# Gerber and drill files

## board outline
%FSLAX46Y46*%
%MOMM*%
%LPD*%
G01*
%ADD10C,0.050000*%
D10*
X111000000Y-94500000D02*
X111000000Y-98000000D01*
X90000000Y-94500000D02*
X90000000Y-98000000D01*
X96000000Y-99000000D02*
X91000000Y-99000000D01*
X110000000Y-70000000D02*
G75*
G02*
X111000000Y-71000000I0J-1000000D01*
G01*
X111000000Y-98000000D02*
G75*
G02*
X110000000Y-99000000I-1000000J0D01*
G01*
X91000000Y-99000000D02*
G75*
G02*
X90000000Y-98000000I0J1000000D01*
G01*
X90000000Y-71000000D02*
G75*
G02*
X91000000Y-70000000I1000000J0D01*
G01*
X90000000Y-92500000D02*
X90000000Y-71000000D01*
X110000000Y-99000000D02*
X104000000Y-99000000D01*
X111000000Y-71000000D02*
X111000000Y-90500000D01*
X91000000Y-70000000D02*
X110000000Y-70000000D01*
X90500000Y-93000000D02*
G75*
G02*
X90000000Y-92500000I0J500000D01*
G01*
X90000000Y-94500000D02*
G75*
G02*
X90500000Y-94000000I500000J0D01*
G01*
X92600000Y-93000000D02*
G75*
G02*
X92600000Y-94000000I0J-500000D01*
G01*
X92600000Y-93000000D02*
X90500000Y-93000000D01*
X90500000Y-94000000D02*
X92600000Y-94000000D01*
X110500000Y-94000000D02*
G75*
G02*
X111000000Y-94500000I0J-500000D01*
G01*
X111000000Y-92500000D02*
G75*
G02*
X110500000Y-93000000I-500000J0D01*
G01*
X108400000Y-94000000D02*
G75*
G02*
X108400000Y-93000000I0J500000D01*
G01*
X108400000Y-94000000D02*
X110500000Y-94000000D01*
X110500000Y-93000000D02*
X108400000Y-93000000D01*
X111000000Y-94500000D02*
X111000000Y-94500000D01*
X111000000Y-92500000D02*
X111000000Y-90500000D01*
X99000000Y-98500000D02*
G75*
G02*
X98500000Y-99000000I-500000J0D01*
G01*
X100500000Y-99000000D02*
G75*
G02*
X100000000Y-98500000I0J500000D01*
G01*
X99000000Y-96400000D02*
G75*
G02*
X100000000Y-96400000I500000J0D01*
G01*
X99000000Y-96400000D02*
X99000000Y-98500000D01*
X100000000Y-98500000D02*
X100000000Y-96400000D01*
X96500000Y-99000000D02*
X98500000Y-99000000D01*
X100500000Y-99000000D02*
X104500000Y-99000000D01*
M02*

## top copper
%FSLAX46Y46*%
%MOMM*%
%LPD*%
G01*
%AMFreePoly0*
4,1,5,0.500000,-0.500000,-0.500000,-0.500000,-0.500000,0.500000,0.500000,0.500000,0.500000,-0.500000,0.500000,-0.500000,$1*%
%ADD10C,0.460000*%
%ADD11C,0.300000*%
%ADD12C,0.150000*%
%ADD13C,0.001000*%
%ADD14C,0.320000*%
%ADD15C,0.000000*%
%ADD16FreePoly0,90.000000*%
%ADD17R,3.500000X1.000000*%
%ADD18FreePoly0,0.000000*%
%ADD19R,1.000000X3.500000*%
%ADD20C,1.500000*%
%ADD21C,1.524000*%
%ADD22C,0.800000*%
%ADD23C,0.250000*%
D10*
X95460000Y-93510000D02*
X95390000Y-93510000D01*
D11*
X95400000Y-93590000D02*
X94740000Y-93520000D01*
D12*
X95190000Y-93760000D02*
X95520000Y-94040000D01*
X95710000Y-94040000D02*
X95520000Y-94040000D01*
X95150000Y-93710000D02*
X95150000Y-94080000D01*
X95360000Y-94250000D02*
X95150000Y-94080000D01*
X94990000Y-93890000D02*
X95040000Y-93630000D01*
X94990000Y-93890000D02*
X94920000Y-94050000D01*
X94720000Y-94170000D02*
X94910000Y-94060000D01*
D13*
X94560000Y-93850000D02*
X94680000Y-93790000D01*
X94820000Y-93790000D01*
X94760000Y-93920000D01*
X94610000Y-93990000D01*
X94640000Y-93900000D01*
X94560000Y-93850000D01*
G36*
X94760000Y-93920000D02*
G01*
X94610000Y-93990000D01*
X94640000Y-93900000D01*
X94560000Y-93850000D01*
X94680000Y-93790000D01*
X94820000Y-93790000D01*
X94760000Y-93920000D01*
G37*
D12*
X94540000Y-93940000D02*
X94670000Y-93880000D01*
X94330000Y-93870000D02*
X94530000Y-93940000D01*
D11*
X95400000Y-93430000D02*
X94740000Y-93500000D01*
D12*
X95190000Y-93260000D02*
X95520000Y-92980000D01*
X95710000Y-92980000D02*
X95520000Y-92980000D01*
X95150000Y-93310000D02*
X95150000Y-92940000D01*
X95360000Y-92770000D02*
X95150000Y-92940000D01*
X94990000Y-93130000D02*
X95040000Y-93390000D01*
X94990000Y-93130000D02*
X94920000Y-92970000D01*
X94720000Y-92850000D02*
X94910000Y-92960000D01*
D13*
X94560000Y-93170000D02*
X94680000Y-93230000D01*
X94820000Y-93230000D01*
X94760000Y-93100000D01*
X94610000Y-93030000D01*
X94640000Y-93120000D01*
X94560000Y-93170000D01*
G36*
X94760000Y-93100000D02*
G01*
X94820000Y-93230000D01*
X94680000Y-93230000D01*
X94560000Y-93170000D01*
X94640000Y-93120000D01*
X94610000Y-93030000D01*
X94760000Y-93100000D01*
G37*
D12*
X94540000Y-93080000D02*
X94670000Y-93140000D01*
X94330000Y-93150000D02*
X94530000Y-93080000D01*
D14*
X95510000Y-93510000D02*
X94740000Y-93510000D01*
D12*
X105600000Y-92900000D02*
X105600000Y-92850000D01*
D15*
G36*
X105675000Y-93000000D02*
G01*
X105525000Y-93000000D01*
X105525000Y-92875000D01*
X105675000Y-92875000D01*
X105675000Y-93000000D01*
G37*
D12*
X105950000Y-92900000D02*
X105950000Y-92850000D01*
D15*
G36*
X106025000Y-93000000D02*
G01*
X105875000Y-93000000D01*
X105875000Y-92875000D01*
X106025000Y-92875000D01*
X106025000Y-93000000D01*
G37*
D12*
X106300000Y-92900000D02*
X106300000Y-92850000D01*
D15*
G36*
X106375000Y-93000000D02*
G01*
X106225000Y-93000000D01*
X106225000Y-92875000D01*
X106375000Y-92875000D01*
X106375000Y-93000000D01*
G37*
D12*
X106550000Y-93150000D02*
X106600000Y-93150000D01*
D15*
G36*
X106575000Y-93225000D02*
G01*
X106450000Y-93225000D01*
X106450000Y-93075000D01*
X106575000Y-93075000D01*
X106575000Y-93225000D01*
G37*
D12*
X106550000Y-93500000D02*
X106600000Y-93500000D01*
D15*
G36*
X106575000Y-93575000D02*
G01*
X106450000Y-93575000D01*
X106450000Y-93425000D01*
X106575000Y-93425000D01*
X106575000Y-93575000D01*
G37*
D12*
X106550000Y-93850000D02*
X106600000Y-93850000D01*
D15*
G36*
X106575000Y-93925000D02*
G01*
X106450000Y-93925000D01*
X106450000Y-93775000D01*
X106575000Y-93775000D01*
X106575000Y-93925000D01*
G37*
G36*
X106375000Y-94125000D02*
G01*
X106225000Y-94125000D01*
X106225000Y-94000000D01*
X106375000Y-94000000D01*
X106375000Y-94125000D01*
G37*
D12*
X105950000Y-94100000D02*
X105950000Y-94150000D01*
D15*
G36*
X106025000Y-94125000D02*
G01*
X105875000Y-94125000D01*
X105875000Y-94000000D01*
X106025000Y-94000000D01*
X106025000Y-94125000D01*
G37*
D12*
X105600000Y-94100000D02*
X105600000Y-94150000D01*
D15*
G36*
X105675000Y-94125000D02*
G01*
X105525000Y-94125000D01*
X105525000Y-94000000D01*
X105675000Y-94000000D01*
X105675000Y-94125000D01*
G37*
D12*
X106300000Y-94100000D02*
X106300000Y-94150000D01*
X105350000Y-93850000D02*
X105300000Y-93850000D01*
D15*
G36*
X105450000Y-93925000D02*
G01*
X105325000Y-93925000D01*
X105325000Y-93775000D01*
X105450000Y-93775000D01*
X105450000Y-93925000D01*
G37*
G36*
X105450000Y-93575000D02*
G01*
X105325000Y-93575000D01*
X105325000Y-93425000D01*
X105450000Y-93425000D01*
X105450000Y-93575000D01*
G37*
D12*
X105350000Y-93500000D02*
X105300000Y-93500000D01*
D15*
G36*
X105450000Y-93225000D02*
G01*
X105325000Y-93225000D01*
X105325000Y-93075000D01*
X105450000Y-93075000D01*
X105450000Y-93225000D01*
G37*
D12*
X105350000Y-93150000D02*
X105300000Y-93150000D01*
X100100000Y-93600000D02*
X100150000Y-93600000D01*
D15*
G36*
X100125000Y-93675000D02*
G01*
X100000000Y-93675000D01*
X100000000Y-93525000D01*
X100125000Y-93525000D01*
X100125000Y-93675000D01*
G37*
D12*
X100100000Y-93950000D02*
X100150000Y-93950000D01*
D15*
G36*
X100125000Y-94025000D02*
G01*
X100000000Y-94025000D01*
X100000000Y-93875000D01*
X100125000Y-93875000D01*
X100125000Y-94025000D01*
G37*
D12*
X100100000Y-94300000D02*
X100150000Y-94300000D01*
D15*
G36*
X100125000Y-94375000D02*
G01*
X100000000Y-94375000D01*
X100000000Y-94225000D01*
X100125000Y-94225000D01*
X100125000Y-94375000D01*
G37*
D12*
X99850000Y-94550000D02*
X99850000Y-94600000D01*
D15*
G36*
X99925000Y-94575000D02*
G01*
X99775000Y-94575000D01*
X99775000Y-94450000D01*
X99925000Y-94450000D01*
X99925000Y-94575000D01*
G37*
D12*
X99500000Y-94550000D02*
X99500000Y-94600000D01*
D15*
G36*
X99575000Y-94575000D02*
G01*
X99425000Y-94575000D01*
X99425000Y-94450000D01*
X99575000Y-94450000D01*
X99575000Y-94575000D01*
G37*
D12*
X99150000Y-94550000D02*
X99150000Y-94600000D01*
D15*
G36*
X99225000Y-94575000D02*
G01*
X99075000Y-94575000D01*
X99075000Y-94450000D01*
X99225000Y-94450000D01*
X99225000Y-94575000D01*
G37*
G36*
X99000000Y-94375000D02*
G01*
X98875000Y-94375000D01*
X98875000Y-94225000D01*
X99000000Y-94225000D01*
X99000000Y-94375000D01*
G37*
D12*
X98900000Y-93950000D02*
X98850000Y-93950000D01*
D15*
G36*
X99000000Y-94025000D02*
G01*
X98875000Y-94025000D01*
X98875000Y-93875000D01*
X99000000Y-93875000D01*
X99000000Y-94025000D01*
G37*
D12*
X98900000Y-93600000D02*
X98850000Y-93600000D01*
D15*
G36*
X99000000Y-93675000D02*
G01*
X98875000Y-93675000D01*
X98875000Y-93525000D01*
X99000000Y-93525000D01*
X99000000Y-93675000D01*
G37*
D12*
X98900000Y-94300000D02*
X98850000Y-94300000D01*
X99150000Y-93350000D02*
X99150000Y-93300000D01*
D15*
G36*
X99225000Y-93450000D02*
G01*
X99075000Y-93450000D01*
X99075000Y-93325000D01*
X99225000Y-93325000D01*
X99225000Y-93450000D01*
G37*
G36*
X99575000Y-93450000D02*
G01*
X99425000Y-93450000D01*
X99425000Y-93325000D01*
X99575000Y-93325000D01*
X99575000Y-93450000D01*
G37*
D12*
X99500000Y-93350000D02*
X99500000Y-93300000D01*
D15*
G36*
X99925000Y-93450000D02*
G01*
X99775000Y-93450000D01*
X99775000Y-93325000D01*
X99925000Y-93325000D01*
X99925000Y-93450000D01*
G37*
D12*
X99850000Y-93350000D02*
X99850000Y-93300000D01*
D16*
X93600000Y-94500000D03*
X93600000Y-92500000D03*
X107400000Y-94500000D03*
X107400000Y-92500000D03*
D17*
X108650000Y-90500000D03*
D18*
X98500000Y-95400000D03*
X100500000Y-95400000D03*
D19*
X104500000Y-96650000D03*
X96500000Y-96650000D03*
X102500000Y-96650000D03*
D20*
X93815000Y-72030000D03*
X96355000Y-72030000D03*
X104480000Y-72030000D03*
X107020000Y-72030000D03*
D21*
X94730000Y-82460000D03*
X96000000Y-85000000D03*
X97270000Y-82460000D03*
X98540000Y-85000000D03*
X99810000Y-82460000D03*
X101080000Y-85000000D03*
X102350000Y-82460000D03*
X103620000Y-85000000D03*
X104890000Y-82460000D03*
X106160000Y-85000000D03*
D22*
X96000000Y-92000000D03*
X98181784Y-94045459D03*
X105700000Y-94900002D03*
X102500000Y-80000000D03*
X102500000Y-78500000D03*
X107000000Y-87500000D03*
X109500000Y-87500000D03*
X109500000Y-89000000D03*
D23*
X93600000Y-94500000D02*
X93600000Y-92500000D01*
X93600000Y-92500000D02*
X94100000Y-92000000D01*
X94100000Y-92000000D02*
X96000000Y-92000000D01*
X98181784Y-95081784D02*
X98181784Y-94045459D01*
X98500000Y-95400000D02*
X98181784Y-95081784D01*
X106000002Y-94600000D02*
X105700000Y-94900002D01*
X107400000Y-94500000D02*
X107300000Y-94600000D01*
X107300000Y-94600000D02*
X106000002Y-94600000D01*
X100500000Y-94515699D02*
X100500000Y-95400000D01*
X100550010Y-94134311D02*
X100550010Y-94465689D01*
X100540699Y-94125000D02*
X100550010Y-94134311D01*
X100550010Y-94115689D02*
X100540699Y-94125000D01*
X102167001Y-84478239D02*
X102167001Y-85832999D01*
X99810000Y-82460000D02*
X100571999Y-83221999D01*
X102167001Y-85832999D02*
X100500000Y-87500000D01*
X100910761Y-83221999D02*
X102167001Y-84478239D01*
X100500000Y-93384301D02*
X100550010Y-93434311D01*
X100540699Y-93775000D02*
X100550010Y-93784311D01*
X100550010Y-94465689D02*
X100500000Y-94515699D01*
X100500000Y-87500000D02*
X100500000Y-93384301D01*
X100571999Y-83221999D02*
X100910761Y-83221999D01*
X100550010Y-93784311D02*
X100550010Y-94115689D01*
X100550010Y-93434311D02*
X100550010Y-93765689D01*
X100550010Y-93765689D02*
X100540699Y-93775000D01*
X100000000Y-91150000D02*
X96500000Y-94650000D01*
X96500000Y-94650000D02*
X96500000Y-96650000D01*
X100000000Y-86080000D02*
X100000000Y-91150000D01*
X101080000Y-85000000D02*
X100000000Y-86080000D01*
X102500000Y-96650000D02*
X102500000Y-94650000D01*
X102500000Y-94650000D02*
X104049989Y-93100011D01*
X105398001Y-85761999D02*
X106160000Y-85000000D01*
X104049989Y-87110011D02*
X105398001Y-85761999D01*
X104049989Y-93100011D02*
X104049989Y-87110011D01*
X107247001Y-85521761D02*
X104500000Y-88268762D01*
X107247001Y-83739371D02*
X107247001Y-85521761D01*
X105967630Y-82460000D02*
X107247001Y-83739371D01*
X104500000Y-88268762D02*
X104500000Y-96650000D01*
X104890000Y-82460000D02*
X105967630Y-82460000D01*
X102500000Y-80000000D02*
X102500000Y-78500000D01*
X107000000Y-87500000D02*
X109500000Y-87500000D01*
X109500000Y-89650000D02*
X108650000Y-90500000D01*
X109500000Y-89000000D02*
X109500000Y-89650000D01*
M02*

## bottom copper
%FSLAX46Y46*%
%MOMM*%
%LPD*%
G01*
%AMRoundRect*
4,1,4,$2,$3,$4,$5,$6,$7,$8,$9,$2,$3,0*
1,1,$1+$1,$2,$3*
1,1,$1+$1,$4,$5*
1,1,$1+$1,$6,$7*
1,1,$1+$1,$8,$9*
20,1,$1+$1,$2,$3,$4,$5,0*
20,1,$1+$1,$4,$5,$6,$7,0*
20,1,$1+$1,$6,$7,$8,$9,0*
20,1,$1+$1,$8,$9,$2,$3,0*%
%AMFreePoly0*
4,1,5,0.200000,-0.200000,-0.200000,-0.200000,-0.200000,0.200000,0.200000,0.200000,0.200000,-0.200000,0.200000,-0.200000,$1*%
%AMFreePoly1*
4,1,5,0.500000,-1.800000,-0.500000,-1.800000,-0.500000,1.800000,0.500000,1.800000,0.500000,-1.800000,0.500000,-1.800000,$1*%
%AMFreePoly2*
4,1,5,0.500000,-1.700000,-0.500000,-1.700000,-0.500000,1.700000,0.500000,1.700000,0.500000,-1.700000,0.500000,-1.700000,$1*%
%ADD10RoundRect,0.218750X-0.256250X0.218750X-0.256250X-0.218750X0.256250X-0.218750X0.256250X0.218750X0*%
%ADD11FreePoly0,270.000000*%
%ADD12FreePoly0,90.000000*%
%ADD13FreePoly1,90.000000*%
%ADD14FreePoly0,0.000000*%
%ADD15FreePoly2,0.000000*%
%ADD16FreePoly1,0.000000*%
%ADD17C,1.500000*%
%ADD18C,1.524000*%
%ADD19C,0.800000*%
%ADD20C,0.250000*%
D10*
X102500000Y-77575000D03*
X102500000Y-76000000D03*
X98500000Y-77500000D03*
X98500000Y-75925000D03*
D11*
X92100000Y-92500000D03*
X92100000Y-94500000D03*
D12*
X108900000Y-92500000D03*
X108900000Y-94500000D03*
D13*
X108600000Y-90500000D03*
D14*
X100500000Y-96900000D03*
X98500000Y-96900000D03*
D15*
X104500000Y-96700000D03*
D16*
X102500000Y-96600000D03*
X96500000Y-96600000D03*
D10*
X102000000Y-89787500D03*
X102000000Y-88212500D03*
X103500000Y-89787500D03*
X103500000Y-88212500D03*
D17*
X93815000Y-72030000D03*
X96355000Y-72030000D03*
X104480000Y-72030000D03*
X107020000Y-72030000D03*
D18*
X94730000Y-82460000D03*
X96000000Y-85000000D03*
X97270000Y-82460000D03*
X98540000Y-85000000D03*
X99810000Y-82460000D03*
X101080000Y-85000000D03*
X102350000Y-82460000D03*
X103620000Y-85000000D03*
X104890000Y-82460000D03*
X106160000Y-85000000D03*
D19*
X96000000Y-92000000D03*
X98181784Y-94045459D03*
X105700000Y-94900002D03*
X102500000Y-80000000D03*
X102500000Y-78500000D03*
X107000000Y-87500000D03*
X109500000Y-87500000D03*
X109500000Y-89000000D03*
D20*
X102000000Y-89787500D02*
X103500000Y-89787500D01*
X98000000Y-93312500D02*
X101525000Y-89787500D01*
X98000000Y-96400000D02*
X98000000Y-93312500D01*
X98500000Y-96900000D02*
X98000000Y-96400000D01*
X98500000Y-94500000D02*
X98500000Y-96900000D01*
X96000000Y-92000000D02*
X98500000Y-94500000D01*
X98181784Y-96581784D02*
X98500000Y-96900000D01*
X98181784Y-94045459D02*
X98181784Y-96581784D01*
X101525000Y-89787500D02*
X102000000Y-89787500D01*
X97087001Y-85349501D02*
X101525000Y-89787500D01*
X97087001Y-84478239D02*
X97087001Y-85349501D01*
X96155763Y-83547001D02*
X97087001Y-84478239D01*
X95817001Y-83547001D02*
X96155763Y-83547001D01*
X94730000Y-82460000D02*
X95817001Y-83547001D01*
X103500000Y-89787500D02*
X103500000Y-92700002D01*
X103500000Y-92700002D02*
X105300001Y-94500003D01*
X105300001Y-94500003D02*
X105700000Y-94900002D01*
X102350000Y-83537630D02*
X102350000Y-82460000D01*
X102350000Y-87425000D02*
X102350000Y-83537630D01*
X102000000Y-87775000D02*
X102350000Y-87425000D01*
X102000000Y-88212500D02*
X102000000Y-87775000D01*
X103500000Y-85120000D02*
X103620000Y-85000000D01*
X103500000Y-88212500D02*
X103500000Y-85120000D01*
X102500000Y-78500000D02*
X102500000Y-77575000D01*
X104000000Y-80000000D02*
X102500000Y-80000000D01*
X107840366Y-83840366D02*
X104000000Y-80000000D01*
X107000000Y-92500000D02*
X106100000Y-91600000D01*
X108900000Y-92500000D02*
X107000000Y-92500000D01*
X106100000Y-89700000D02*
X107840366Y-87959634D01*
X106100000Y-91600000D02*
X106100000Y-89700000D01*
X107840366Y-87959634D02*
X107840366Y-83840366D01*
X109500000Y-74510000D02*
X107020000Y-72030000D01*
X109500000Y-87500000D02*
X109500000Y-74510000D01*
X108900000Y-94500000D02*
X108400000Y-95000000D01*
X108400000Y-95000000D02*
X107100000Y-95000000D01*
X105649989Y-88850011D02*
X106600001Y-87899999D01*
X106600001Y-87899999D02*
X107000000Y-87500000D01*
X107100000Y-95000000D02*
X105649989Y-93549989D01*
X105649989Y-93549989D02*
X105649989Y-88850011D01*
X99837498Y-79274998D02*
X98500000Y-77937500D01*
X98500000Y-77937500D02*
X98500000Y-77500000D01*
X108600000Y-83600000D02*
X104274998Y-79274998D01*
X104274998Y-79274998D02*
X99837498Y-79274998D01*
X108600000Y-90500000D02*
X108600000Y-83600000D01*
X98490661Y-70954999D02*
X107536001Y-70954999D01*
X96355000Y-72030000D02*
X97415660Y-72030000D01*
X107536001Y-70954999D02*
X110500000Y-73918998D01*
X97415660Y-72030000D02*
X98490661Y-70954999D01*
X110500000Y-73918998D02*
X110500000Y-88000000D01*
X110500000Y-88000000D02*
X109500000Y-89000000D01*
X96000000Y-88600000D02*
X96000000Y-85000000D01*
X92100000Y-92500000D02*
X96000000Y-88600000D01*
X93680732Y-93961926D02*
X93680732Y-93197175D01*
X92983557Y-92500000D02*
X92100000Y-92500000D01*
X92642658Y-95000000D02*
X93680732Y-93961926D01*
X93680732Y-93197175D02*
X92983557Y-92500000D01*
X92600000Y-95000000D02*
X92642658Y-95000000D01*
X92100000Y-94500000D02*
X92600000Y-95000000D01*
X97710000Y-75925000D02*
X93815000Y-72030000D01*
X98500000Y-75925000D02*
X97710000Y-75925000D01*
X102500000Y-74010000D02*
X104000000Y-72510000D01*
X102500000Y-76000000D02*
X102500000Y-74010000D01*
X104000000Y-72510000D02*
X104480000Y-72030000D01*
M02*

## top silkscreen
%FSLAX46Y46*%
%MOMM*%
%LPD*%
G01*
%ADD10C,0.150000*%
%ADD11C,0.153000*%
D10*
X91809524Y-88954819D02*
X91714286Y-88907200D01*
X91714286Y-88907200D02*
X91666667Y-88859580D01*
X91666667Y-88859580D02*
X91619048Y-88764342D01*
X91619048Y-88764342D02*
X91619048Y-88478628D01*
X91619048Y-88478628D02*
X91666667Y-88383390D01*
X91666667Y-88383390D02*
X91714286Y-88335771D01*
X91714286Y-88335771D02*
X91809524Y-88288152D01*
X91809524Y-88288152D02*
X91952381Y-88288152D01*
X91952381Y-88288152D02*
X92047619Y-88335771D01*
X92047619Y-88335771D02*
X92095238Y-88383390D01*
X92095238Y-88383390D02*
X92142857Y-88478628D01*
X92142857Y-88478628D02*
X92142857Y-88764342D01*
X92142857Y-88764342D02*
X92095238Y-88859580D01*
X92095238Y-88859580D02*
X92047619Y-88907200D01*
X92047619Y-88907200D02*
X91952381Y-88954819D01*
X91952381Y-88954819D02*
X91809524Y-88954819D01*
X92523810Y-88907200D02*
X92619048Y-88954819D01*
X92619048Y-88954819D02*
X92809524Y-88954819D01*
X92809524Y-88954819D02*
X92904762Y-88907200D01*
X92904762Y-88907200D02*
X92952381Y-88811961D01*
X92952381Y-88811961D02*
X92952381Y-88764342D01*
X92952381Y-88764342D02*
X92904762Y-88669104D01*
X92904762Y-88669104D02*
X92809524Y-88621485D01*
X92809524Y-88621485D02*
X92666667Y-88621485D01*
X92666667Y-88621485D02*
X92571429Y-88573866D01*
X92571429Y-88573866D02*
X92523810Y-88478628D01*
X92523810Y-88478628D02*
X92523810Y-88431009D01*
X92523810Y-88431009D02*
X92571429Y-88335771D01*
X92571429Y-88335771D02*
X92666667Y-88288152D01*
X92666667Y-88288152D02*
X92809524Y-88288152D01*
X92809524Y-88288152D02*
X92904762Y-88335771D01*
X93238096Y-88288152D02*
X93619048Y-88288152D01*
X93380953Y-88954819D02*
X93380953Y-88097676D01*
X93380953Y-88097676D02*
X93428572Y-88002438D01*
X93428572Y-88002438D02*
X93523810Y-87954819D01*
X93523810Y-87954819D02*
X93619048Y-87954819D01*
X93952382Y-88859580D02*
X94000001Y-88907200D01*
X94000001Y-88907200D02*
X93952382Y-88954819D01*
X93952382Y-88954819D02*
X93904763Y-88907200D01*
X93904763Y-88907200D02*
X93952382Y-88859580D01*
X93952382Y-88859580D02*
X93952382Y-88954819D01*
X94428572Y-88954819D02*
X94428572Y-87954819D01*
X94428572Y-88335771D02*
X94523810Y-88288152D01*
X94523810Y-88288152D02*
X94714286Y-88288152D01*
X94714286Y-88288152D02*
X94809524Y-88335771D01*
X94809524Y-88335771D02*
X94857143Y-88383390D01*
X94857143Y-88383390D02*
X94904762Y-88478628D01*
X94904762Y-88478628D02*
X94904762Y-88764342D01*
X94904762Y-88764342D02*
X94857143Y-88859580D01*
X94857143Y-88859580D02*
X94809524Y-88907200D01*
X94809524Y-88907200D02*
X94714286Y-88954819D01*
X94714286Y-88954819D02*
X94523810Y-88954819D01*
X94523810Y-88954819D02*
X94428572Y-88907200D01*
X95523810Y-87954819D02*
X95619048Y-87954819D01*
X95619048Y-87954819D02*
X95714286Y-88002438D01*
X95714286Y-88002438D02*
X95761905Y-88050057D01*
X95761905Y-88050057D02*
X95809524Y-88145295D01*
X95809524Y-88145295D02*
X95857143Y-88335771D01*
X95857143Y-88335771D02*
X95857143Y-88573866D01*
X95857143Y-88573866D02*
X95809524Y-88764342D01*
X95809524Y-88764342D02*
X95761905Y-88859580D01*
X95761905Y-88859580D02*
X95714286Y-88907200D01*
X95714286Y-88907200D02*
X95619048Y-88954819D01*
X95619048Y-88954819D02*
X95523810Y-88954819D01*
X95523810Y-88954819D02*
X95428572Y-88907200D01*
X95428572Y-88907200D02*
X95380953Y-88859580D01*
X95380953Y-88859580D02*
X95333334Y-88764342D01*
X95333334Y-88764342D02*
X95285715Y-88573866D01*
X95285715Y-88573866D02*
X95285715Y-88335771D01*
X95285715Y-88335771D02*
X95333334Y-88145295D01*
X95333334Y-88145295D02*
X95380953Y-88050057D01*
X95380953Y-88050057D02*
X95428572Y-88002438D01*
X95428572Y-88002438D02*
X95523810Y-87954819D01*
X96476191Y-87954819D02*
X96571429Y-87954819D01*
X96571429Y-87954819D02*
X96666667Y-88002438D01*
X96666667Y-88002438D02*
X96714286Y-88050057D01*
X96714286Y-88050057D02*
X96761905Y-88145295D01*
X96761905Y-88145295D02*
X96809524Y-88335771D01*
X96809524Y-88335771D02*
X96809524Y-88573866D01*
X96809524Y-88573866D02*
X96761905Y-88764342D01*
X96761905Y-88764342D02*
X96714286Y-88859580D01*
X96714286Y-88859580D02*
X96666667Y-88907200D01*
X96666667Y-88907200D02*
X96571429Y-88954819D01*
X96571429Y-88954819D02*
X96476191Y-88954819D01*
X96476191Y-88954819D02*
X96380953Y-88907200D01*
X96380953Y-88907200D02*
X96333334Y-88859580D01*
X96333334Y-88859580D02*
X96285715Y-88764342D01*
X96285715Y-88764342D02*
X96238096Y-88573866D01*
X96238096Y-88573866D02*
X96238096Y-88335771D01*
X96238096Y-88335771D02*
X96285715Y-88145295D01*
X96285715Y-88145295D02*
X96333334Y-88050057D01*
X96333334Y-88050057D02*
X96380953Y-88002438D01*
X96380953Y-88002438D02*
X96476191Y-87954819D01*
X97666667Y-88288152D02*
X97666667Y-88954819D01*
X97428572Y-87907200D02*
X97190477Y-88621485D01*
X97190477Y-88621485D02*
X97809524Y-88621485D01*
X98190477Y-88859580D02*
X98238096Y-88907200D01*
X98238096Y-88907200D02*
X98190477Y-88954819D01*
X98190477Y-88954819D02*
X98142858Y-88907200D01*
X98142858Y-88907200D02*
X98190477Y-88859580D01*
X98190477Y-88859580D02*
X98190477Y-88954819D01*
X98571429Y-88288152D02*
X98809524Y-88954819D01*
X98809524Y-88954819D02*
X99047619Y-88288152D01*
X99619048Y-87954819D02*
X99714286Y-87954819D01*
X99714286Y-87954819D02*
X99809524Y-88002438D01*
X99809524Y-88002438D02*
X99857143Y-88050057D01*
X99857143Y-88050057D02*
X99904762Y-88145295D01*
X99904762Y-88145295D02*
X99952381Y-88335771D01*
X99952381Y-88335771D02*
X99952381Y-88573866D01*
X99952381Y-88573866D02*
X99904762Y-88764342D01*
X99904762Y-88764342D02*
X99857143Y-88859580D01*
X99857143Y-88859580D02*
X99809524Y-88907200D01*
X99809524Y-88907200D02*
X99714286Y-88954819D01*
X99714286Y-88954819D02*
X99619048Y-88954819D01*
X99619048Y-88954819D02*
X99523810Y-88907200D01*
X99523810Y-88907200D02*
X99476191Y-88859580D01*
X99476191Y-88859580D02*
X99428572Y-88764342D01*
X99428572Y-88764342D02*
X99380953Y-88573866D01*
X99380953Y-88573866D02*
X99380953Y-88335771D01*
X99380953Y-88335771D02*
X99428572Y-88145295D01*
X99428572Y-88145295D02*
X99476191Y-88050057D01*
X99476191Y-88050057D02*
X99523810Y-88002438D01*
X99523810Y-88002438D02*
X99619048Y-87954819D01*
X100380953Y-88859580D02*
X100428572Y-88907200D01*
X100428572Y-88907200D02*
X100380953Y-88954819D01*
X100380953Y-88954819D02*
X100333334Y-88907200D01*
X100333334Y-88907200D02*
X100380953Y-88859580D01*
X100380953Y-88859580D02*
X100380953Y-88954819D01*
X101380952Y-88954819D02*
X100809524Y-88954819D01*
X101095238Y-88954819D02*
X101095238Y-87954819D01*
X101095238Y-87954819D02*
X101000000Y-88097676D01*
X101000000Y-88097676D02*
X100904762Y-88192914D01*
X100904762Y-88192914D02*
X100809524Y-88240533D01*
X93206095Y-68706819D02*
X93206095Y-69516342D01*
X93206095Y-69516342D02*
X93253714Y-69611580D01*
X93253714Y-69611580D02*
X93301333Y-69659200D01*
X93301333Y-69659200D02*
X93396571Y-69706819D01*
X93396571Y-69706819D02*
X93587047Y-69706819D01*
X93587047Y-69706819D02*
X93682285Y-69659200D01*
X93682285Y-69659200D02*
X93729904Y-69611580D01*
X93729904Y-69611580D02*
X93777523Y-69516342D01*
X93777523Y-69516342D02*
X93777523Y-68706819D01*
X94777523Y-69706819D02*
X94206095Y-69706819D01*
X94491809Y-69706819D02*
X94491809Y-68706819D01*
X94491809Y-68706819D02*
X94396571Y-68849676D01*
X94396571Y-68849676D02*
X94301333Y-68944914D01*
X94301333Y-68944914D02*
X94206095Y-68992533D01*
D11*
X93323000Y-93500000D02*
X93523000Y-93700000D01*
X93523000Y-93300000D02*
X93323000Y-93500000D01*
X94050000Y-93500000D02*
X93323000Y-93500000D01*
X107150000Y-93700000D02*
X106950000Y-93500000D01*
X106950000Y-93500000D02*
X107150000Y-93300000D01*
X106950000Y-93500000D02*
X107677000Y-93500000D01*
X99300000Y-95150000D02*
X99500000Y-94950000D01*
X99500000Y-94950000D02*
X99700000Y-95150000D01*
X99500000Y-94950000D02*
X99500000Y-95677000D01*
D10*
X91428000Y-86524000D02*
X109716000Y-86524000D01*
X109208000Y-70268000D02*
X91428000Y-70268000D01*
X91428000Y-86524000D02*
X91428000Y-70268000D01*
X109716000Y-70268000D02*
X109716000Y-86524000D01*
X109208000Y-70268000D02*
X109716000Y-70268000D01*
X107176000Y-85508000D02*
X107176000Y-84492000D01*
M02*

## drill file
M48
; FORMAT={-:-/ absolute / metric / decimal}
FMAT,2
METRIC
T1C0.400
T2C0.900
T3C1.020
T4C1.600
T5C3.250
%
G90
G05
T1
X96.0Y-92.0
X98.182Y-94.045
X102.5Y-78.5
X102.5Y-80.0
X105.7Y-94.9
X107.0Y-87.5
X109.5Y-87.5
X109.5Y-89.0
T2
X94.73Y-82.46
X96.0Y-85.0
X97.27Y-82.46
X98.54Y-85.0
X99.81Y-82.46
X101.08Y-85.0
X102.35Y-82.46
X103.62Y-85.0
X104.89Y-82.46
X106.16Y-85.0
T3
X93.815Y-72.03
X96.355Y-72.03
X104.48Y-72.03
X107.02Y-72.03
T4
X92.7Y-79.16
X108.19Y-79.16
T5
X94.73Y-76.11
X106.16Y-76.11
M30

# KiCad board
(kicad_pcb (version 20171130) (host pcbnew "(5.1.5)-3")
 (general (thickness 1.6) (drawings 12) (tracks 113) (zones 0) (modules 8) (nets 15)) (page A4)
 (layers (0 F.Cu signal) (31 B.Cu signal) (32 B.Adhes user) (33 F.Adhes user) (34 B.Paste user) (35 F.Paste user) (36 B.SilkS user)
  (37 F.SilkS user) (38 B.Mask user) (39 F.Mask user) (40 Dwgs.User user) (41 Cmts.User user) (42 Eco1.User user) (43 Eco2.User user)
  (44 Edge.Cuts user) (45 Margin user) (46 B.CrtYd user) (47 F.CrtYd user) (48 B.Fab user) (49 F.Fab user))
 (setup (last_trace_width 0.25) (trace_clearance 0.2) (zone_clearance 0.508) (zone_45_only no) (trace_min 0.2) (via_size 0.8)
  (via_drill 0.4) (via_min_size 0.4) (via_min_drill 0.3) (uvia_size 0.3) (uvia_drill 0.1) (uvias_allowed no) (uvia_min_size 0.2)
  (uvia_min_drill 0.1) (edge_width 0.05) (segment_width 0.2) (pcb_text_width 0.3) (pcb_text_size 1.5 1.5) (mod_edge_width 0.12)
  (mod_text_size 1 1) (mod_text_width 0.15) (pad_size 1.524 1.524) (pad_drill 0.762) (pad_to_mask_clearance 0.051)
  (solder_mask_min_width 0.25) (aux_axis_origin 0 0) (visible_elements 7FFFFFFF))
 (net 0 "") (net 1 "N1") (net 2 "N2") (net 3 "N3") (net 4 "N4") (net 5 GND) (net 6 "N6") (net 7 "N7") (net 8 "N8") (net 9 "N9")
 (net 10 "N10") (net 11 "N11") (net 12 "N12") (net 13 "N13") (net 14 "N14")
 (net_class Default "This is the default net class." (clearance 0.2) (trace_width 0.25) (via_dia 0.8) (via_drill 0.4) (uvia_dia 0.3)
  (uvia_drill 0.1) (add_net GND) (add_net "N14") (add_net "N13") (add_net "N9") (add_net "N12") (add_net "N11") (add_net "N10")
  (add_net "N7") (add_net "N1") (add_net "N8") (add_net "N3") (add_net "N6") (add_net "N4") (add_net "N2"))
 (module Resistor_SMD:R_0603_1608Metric (layer B.Cu) (at 102.5 76.7875 270)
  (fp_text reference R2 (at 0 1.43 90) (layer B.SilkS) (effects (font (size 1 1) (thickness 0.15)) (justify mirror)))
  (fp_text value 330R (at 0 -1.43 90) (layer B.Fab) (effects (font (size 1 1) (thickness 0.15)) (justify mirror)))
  (pad 2 smd roundrect (at 0.7875 0 270) (size 0.875 0.95) (layers B.Cu B.Paste B.Mask) (roundrect_rratio 0.25) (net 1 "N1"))
  (pad 1 smd roundrect (at -0.7875 0 270) (size 0.875 0.95) (layers B.Cu B.Paste B.Mask) (roundrect_rratio 0.25) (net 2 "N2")))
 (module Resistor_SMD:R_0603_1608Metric (layer B.Cu) (at 98.5 76.7125 270)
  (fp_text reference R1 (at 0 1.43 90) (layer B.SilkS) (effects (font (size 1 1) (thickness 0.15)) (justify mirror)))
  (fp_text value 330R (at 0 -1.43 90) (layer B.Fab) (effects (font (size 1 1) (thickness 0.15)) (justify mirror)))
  (pad 2 smd roundrect (at 0.7875 0 270) (size 0.875 0.95) (layers B.Cu B.Paste B.Mask) (roundrect_rratio 0.25) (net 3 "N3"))
  (pad 1 smd roundrect (at -0.7875 0 270) (size 0.875 0.95) (layers B.Cu B.Paste B.Mask) (roundrect_rratio 0.25) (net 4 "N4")))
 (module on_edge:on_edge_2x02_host (layer F.Cu) (at 90 92.5 90)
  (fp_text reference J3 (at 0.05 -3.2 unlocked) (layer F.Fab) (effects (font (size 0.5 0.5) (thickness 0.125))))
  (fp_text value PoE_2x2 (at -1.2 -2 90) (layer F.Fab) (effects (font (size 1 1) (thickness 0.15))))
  (fp_arc (start 0 0.5) (end 0 0) (angle -90) (layer Edge.Cuts) (width 0.05))
  (fp_arc (start -2 0.5) (end -1.5 0.5) (angle -90) (layer Edge.Cuts) (width 0.05))
  (fp_arc (start -1 2.6) (end -1.5 2.6) (angle -180) (layer Edge.Cuts) (width 0.05))
  (fp_line (start -1.01 5.46) (end -1.01 5.39) (layer F.Cu) (width 0.46))
  (fp_line (start -1.09 5.4) (end -1.02 4.74) (layer F.Cu) (width 0.3))
  (fp_line (start -1.26 5.19) (end -1.54 5.52) (layer F.Cu) (width 0.15))
  (fp_line (start -1.54 5.71) (end -1.54 5.52) (layer F.Cu) (width 0.15))
  (fp_line (start -1.21 5.15) (end -1.58 5.15) (layer F.Cu) (width 0.15))
  (fp_line (start -1.75 5.36) (end -1.58 5.15) (layer F.Cu) (width 0.15))
  (fp_line (start -1.39 4.99) (end -1.13 5.04) (layer F.Cu) (width 0.15))
  (fp_line (start -1.39 4.99) (end -1.55 4.92) (layer F.Cu) (width 0.15))
  (fp_line (start -1.67 4.72) (end -1.56 4.91) (layer F.Cu) (width 0.15))
  (fp_poly (pts (xy -1.35 4.56) (xy -1.29 4.68) (xy -1.29 4.82) (xy -1.42 4.76) (xy -1.49 4.61) (xy -1.4 4.64)) (layer F.Cu) (width 0.001))
  (fp_line (start -1.44 4.54) (end -1.38 4.67) (layer F.Cu) (width 0.15))
  (fp_line (start -1.37 4.33) (end -1.44 4.53) (layer F.Cu) (width 0.15))
  (fp_line (start -0.5 2.6) (end -0.5 0.5) (layer Edge.Cuts) (width 0.05))
  (fp_line (start -1.5 0.5) (end -1.5 2.6) (layer Edge.Cuts) (width 0.05))
  (fp_line (start -1 3.323) (end -1.2 3.523) (layer F.SilkS) (width 0.153))
  (fp_line (start -0.8 3.523) (end -1 3.323) (layer F.SilkS) (width 0.153))
  (fp_line (start -1 4.05) (end -1 3.323) (layer F.SilkS) (width 0.153))
  (fp_line (start -0.93 5.4) (end -1 4.74) (layer F.Cu) (width 0.3))
  (fp_line (start -0.76 5.19) (end -0.48 5.52) (layer F.Cu) (width 0.15))
  (fp_line (start -0.48 5.71) (end -0.48 5.52) (layer F.Cu) (width 0.15))
  (fp_line (start -0.81 5.15) (end -0.44 5.15) (layer F.Cu) (width 0.15))
  (fp_line (start -0.27 5.36) (end -0.44 5.15) (layer F.Cu) (width 0.15))
  (fp_line (start -0.63 4.99) (end -0.89 5.04) (layer F.Cu) (width 0.15))
  (fp_line (start -0.63 4.99) (end -0.47 4.92) (layer F.Cu) (width 0.15))
  (fp_line (start -0.35 4.72) (end -0.46 4.91) (layer F.Cu) (width 0.15))
  (fp_poly (pts (xy -0.67 4.56) (xy -0.73 4.68) (xy -0.73 4.82) (xy -0.6 4.76) (xy -0.53 4.61) (xy -0.62 4.64)) (layer F.Cu) (width 0.001))
  (fp_line (start -0.58 4.54) (end -0.64 4.67) (layer F.Cu) (width 0.15))
  (fp_line (start -0.65 4.33) (end -0.58 4.53) (layer F.Cu) (width 0.15))
  (fp_line (start -1.01 5.51) (end -1.01 4.74) (layer F.Cu) (width 0.32))
  (pad 1 smd custom (at -2 3.6 90) (size 1 1) (layers F.Cu F.Mask) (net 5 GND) (zone_connect 0) (options (clearance outline) (anchor rect))
   (primitives))
  (pad 2 smd custom (at 0 3.6 90) (size 1 1) (layers F.Cu F.Mask) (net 5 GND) (zone_connect 0) (options (clearance outline) (anchor rect))
   (primitives))
  (pad 4 smd custom (at 0 2.1 270) (size 0.4 0.4) (layers B.Cu B.Mask) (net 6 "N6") (zone_connect 0)
   (options (clearance outline) (anchor rect)) (primitives))
  (pad 3 smd custom (at -2 2.1 270) (size 0.4 0.4) (layers B.Cu B.Mask) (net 6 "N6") (zone_connect 0)
   (options (clearance outline) (anchor rect)) (primitives)))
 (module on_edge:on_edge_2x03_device (layer F.Cu) (at 111 92.5 90)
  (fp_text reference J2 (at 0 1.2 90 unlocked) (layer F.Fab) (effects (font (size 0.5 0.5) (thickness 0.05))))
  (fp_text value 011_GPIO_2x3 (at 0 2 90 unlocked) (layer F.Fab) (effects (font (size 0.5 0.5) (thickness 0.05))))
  (fp_arc (start -2 -0.5) (end -2 0) (angle -90) (layer Edge.Cuts) (width 0.05))
  (fp_arc (start 0 -0.5) (end -0.5 -0.5) (angle -90) (layer Edge.Cuts) (width 0.05))
  (fp_arc (start -1 -2.6) (end -0.5 -2.6) (angle -180) (layer Edge.Cuts) (width 0.05))
  (fp_line (start -0.4 -5.4) (end -0.35 -5.4) (layer F.Cu) (width 0.15))
  (fp_poly (pts (xy -0.5 -5.325) (xy -0.5 -5.475) (xy -0.375 -5.475) (xy -0.375 -5.325)) (layer F.Cu) (width 0))
  (fp_line (start -0.4 -5.05) (end -0.35 -5.05) (layer F.Cu) (width 0.15))
  (fp_poly (pts (xy -0.5 -4.975) (xy -0.5 -5.125) (xy -0.375 -5.125) (xy -0.375 -4.975)) (layer F.Cu) (width 0))
  (fp_line (start -0.4 -4.7) (end -0.35 -4.7) (layer F.Cu) (width 0.15))
  (fp_poly (pts (xy -0.5 -4.625) (xy -0.5 -4.775) (xy -0.375 -4.775) (xy -0.375 -4.625)) (layer F.Cu) (width 0))
  (fp_line (start -0.65 -4.45) (end -0.65 -4.4) (layer F.Cu) (width 0.15))
  (fp_poly (pts (xy -0.725 -4.55) (xy -0.575 -4.55) (xy -0.575 -4.425) (xy -0.725 -4.425)) (layer F.Cu) (width 0))
  (fp_line (start -1 -4.45) (end -1 -4.4) (layer F.Cu) (width 0.15))
  (fp_poly (pts (xy -1.075 -4.55) (xy -0.925 -4.55) (xy -0.925 -4.425) (xy -1.075 -4.425)) (layer F.Cu) (width 0))
  (fp_line (start -1.35 -4.45) (end -1.35 -4.4) (layer F.Cu) (width 0.15))
  (fp_poly (pts (xy -1.425 -4.55) (xy -1.275 -4.55) (xy -1.275 -4.425) (xy -1.425 -4.425)) (layer F.Cu) (width 0))
  (fp_poly (pts (xy -1.5 -4.775) (xy -1.5 -4.625) (xy -1.625 -4.625) (xy -1.625 -4.775)) (layer F.Cu) (width 0))
  (fp_line (start -1.6 -5.05) (end -1.65 -5.05) (layer F.Cu) (width 0.15))
  (fp_poly (pts (xy -1.5 -5.125) (xy -1.5 -4.975) (xy -1.625 -4.975) (xy -1.625 -5.125)) (layer F.Cu) (width 0))
  (fp_line (start -1.6 -5.4) (end -1.65 -5.4) (layer F.Cu) (width 0.15))
  (fp_poly (pts (xy -1.5 -5.475) (xy -1.5 -5.325) (xy -1.625 -5.325) (xy -1.625 -5.475)) (layer F.Cu) (width 0))
  (fp_line (start -1.6 -4.7) (end -1.65 -4.7) (layer F.Cu) (width 0.15))
  (fp_line (start -1.5 -2.6) (end -1.5 -0.5) (layer Edge.Cuts) (width 0.05))
  (fp_line (start -0.5 -0.5) (end -0.5 -2.6) (layer Edge.Cuts) (width 0.05))
  (fp_line (start -1.2 -3.85) (end -1 -4.05) (layer F.SilkS) (width 0.153))
  (fp_line (start -1 -4.05) (end -0.8 -3.85) (layer F.SilkS) (width 0.153))
  (fp_line (start -1 -4.05) (end -1 -3.323) (layer F.SilkS) (width 0.153))
  (fp_line (start -2 0) (end -2 0) (layer Edge.Cuts) (width 0.05))
  (fp_line (start 0 0) (end 2 0) (layer Edge.Cuts) (width 0.05))
  (fp_line (start -1.35 -5.65) (end -1.35 -5.7) (layer F.Cu) (width 0.15))
  (fp_poly (pts (xy -1.275 -5.55) (xy -1.425 -5.55) (xy -1.425 -5.675) (xy -1.275 -5.675)) (layer F.Cu) (width 0))
  (fp_poly (pts (xy -0.925 -5.55) (xy -1.075 -5.55) (xy -1.075 -5.675) (xy -0.925 -5.675)) (layer F.Cu) (width 0))
  (fp_line (start -1 -5.65) (end -1 -5.7) (layer F.Cu) (width 0.15))
  (fp_poly (pts (xy -0.575 -5.55) (xy -0.725 -5.55) (xy -0.725 -5.675) (xy -0.575 -5.675)) (layer F.Cu) (width 0))
  (fp_line (start -0.65 -5.65) (end -0.65 -5.7) (layer F.Cu) (width 0.15))
  (pad 1 smd custom (at -2 -3.6 90) (size 1 1) (layers F.Cu F.Mask) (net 5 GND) (zone_connect 0) (options (clearance outline) (anchor rect))
   (primitives))
  (pad 2 smd custom (at 0 -3.6 90) (size 1 1) (layers F.Cu F.Mask) (zone_connect 0) (options (clearance outline) (anchor rect)) (primitives))
  (pad 4 smd custom (at 0 -2.1 90) (size 0.4 0.4) (layers B.Cu B.Mask) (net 1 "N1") (zone_connect 0)
   (options (clearance outline) (anchor rect)) (primitives))
  (pad 3 smd custom (at -2 -2.1 90) (size 0.4 0.4) (layers B.Cu B.Mask) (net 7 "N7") (zone_connect 0)
   (options (clearance outline) (anchor rect)) (primitives))
  (pad 6 smd custom (at 2 -2.4 90) (size 1 3.6) (layers B.Cu B.Mask) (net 3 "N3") (zone_connect 0)
   (options (clearance outline) (anchor rect)) (primitives))
  (pad 5 smd rect (at 2 -2.35 270) (size 1 3.5) (layers F.Cu F.Mask) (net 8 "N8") (zone_connect 0)))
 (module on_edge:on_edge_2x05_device (layer F.Cu) (at 100.5 99)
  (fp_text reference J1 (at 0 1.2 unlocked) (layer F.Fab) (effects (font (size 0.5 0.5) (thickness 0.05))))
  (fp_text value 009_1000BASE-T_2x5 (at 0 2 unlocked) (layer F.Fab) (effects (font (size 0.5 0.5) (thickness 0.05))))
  (fp_arc (start -2 -0.5) (end -2 0) (angle -90) (layer Edge.Cuts) (width 0.05))
  (fp_arc (start 0 -0.5) (end -0.5 -0.5) (angle -90) (layer Edge.Cuts) (width 0.05))
  (fp_arc (start -1 -2.6) (end -0.5 -2.6) (angle -180) (layer Edge.Cuts) (width 0.05))
  (fp_line (start -0.4 -5.4) (end -0.35 -5.4) (layer F.Cu) (width 0.15))
  (fp_poly (pts (xy -0.5 -5.325) (xy -0.5 -5.475) (xy -0.375 -5.475) (xy -0.375 -5.325)) (layer F.Cu) (width 0))
  (fp_line (start -0.4 -5.05) (end -0.35 -5.05) (layer F.Cu) (width 0.15))
  (fp_poly (pts (xy -0.5 -4.975) (xy -0.5 -5.125) (xy -0.375 -5.125) (xy -0.375 -4.975)) (layer F.Cu) (width 0))
  (fp_line (start -0.4 -4.7) (end -0.35 -4.7) (layer F.Cu) (width 0.15))
  (fp_poly (pts (xy -0.5 -4.625) (xy -0.5 -4.775) (xy -0.375 -4.775) (xy -0.375 -4.625)) (layer F.Cu) (width 0))
  (fp_line (start -0.65 -4.45) (end -0.65 -4.4) (layer F.Cu) (width 0.15))
  (fp_poly (pts (xy -0.725 -4.55) (xy -0.575 -4.55) (xy -0.575 -4.425) (xy -0.725 -4.425)) (layer F.Cu) (width 0))
  (fp_line (start -1 -4.45) (end -1 -4.4) (layer F.Cu) (width 0.15))
  (fp_poly (pts (xy -1.075 -4.55) (xy -0.925 -4.55) (xy -0.925 -4.425) (xy -1.075 -4.425)) (layer F.Cu) (width 0))
  (fp_line (start -1.35 -4.45) (end -1.35 -4.4) (layer F.Cu) (width 0.15))
  (fp_poly (pts (xy -1.425 -4.55) (xy -1.275 -4.55) (xy -1.275 -4.425) (xy -1.425 -4.425)) (layer F.Cu) (width 0))
  (fp_poly (pts (xy -1.5 -4.775) (xy -1.5 -4.625) (xy -1.625 -4.625) (xy -1.625 -4.775)) (layer F.Cu) (width 0))
  (fp_line (start -1.6 -5.05) (end -1.65 -5.05) (layer F.Cu) (width 0.15))
  (fp_poly (pts (xy -1.5 -5.125) (xy -1.5 -4.975) (xy -1.625 -4.975) (xy -1.625 -5.125)) (layer F.Cu) (width 0))
  (fp_line (start -1.6 -5.4) (end -1.65 -5.4) (layer F.Cu) (width 0.15))
  (fp_poly (pts (xy -1.5 -5.475) (xy -1.5 -5.325) (xy -1.625 -5.325) (xy -1.625 -5.475)) (layer F.Cu) (width 0))
  (fp_line (start -1.6 -4.7) (end -1.65 -4.7) (layer F.Cu) (width 0.15))
  (fp_line (start -1.5 -2.6) (end -1.5 -0.5) (layer Edge.Cuts) (width 0.05))
  (fp_line (start -0.5 -0.5) (end -0.5 -2.6) (layer Edge.Cuts) (width 0.05))
  (fp_line (start -1.2 -3.85) (end -1 -4.05) (layer F.SilkS) (width 0.153))
  (fp_line (start -1 -4.05) (end -0.8 -3.85) (layer F.SilkS) (width 0.153))
  (fp_line (start -1 -4.05) (end -1 -3.323) (layer F.SilkS) (width 0.153))
  (fp_line (start -4 0) (end -2 0) (layer Edge.Cuts) (width 0.05))
  (fp_line (start 0 0) (end 4 0) (layer Edge.Cuts) (width 0.05))
  (fp_line (start -1.35 -5.65) (end -1.35 -5.7) (layer F.Cu) (width 0.15))
  (fp_poly (pts (xy -1.275 -5.55) (xy -1.425 -5.55) (xy -1.425 -5.675) (xy -1.275 -5.675)) (layer F.Cu) (width 0))
  (fp_poly (pts (xy -0.925 -5.55) (xy -1.075 -5.55) (xy -1.075 -5.675) (xy -0.925 -5.675)) (layer F.Cu) (width 0))
  (fp_line (start -1 -5.65) (end -1 -5.7) (layer F.Cu) (width 0.15))
  (fp_poly (pts (xy -0.575 -5.55) (xy -0.725 -5.55) (xy -0.725 -5.675) (xy -0.575 -5.675)) (layer F.Cu) (width 0))
  (fp_line (start -0.65 -5.65) (end -0.65 -5.7) (layer F.Cu) (width 0.15))
  (pad 1 smd custom (at -2 -3.6) (size 1 1) (layers F.Cu F.Mask) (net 5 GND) (zone_connect 0) (options (clearance outline) (anchor rect))
   (primitives))
  (pad 2 smd custom (at 0 -3.6) (size 1 1) (layers F.Cu F.Mask) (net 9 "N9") (zone_connect 0) (options (clearance outline) (anchor rect))
   (primitives))
  (pad 4 smd custom (at 0 -2.1) (size 0.4 0.4) (layers B.Cu B.Mask) (zone_connect 0) (options (clearance outline) (anchor rect))
   (primitives))
  (pad 3 smd custom (at -2 -2.1) (size 0.4 0.4) (layers B.Cu B.Mask) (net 5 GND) (zone_connect 0)
   (options (clearance outline) (anchor rect)) (primitives))
  (pad 10 smd custom (at 4 -2.3) (size 1 3.4) (layers B.Cu B.Mask) (zone_connect 0) (options (clearance outline) (anchor rect)) (primitives))
  (pad 6 smd custom (at 2 -2.4) (size 1 3.6) (layers B.Cu B.Mask) (zone_connect 0) (options (clearance outline) (anchor rect)) (primitives))
  (pad 8 smd custom (at -4 -2.4) (size 1 3.6) (layers B.Cu B.Mask) (zone_connect 0) (options (clearance outline) (anchor rect)) (primitives))
  (pad 9 smd rect (at 4 -2.35 180) (size 1 3.5) (layers F.Cu F.Mask) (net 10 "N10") (zone_connect 0))
  (pad 7 smd rect (at -4 -2.35 180) (size 1 3.5) (layers F.Cu F.Mask) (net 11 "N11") (zone_connect 0))
  (pad 5 smd rect (at 2 -2.35 180) (size 1 3.5) (layers F.Cu F.Mask) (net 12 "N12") (zone_connect 0)))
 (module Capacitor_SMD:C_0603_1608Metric (layer B.Cu) (at 102 89 270)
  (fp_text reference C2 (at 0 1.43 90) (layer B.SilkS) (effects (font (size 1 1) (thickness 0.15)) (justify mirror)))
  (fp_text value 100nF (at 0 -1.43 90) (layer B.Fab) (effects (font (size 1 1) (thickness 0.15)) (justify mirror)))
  (pad 2 smd roundrect (at 0.7875 0 270) (size 0.875 0.95) (layers B.Cu B.Paste B.Mask) (roundrect_rratio 0.25) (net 5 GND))
  (pad 1 smd roundrect (at -0.7875 0 270) (size 0.875 0.95) (layers B.Cu B.Paste B.Mask) (roundrect_rratio 0.25) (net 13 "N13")))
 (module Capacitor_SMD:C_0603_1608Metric (layer B.Cu) (at 103.5 89 270)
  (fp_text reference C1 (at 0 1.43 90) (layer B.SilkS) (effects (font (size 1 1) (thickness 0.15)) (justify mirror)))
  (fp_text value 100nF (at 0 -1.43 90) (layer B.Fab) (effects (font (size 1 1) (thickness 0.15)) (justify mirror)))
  (pad 2 smd roundrect (at 0.7875 0 270) (size 0.875 0.95) (layers B.Cu B.Paste B.Mask) (roundrect_rratio 0.25) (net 5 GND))
  (pad 1 smd roundrect (at -0.7875 0 270) (size 0.875 0.95) (layers B.Cu B.Paste B.Mask) (roundrect_rratio 0.25) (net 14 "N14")))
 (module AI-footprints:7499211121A (layer F.Cu) (at 96 85)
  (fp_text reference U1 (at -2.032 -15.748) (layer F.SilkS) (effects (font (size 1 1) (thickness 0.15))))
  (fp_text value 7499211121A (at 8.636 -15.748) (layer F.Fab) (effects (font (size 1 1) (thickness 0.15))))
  (fp_line (start -4.572 1.524) (end 13.716 1.524) (layer F.SilkS) (width 0.15))
  (fp_line (start 13.208 -14.732) (end -4.572 -14.732) (layer F.SilkS) (width 0.15))
  (fp_line (start -4.572 1.524) (end -4.572 -14.732) (layer F.SilkS) (width 0.15))
  (fp_line (start 13.716 -14.732) (end 13.716 1.524) (layer F.SilkS) (width 0.15))
  (fp_line (start 13.208 -14.732) (end 13.716 -14.732) (layer F.SilkS) (width 0.15))
  (fp_line (start 11.176 0.508) (end 11.176 -0.508) (layer F.SilkS) (width 0.15))
  (pad 14 thru_hole circle (at -2.185 -12.97) (size 1.5 1.5) (drill 1.02) (layers *.Cu *.Mask) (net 4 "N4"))
  (pad 13 thru_hole circle (at 0.355 -12.97) (size 1.5 1.5) (drill 1.02) (layers *.Cu *.Mask) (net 8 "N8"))
  (pad 12 thru_hole circle (at 8.48 -12.97) (size 1.5 1.5) (drill 1.02) (layers *.Cu *.Mask) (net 2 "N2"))
  (pad 11 thru_hole circle (at 11.02 -12.97) (size 1.5 1.5) (drill 1.02) (layers *.Cu *.Mask) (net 7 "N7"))
  (pad "" np_thru_hole circle (at 12.19 -5.84) (size 1.6 1.6) (drill 1.6) (layers *.Cu *.Mask))
  (pad "" np_thru_hole circle (at -3.3 -5.84) (size 1.6 1.6) (drill 1.6) (layers *.Cu *.Mask))
  (pad "" np_thru_hole circle (at 10.16 -8.89) (size 3.25 3.25) (drill 3.25) (layers *.Cu *.Mask))
  (pad "" np_thru_hole circle (at -1.27 -8.89) (size 3.25 3.25) (drill 3.25) (layers *.Cu *.Mask))
  (pad 10 thru_hole circle (at -1.27 -2.54) (size 1.524 1.524) (drill 0.9) (layers *.Cu *.Mask) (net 5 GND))
  (pad 9 thru_hole circle (at 0 0) (size 1.524 1.524) (drill 0.9) (layers *.Cu *.Mask) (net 6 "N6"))
  (pad 8 thru_hole circle (at 1.27 -2.54) (size 1.524 1.524) (drill 0.9) (layers *.Cu *.Mask))
  (pad 7 thru_hole circle (at 2.54 0) (size 1.524 1.524) (drill 0.9) (layers *.Cu *.Mask))
  (pad 6 thru_hole circle (at 3.81 -2.54) (size 1.524 1.524) (drill 0.9) (layers *.Cu *.Mask) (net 9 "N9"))
  (pad 5 thru_hole circle (at 5.08 0) (size 1.524 1.524) (drill 0.9) (layers *.Cu *.Mask) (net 11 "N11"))
  (pad 4 thru_hole circle (at 6.35 -2.54) (size 1.524 1.524) (drill 0.9) (layers *.Cu *.Mask) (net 13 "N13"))
  (pad 3 thru_hole circle (at 7.62 0) (size 1.524 1.524) (drill 0.9) (layers *.Cu *.Mask) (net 14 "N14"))
  (pad 2 thru_hole circle (at 8.89 -2.54) (size 1.524 1.524) (drill 0.9) (layers *.Cu *.Mask) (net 10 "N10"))
  (pad 1 thru_hole circle (at 10.16 0) (size 1.524 1.524) (drill 0.9) (layers *.Cu *.Mask) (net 12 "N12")))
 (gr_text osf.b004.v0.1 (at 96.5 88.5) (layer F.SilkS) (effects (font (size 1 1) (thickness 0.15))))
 (gr_line (start 111 94.5) (end 111 98) (layer Edge.Cuts) (width 0.05))
 (gr_line (start 90 94.5) (end 90 98) (layer Edge.Cuts) (width 0.05))
 (gr_line (start 96 99) (end 91 99) (layer Edge.Cuts) (width 0.05))
 (gr_arc (start 110 71) (end 111 71) (angle -90) (layer Edge.Cuts) (width 0.05))
 (gr_arc (start 110 98) (end 110 99) (angle -90) (layer Edge.Cuts) (width 0.05))
 (gr_arc (start 91 98) (end 90 98) (angle -90) (layer Edge.Cuts) (width 0.05))
 (gr_arc (start 91 71) (end 91 70) (angle -90) (layer Edge.Cuts) (width 0.05))
 (gr_line (start 90 92.5) (end 90 71) (layer Edge.Cuts) (width 0.05))
 (gr_line (start 110 99) (end 104 99) (layer Edge.Cuts) (width 0.05))
 (gr_line (start 111 71) (end 111 90.5) (layer Edge.Cuts) (width 0.05))
 (gr_line (start 91 70) (end 110 70) (layer Edge.Cuts) (width 0.05))
 (segment (start 102 89.7875) (end 103.5 89.7875) (width 0.25) (layer B.Cu) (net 5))
 (segment (start 98 93.3125) (end 101.525 89.7875) (width 0.25) (layer B.Cu) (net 5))
 (segment (start 98 96.4) (end 98 93.3125) (width 0.25) (layer B.Cu) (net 5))
 (segment (start 98.5 96.9) (end 98 96.4) (width 0.25) (layer B.Cu) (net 5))
 (segment (start 93.6 94.5) (end 93.6 92.5) (width 0.25) (layer F.Cu) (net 5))
 (via (at 96 92) (size 0.8) (drill 0.4) (layers F.Cu B.Cu) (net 5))
 (segment (start 93.6 92.5) (end 94.1 92) (width 0.25) (layer F.Cu) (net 5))
 (segment (start 94.1 92) (end 96 92) (width 0.25) (layer F.Cu) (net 5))
 (segment (start 98.5 94.5) (end 98.5 96.9) (width 0.25) (layer B.Cu) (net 5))
 (segment (start 96 92) (end 98.5 94.5) (width 0.25) (layer B.Cu) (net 5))
 (via (at 98.181784 94.045459) (size 0.8) (drill 0.4) (layers F.Cu B.Cu) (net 5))
 (segment (start 98.181784 95.081784) (end 98.181784 94.045459) (width 0.25) (layer F.Cu) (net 5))
 (segment (start 98.5 95.4) (end 98.181784 95.081784) (width 0.25) (layer F.Cu) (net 5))
 (segment (start 98.181784 96.581784) (end 98.5 96.9) (width 0.25) (layer B.Cu) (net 5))
 (segment (start 98.181784 94.045459) (end 98.181784 96.581784) (width 0.25) (layer B.Cu) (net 5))
 (segment (start 101.525 89.7875) (end 102 89.7875) (width 0.25) (layer B.Cu) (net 5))
 (segment (start 97.087001 85.349501) (end 101.525 89.7875) (width 0.25) (layer B.Cu) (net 5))
 (segment (start 97.087001 84.478239) (end 97.087001 85.349501) (width 0.25) (layer B.Cu) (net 5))
 (segment (start 96.155763 83.547001) (end 97.087001 84.478239) (width 0.25) (layer B.Cu) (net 5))
 (segment (start 95.817001 83.547001) (end 96.155763 83.547001) (width 0.25) (layer B.Cu) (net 5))
 (segment (start 94.73 82.46) (end 95.817001 83.547001) (width 0.25) (layer B.Cu) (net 5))
 (via (at 105.7 94.900002) (size 0.8) (drill 0.4) (layers F.Cu B.Cu) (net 5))
 (segment (start 103.5 89.7875) (end 103.5 92.700002) (width 0.25) (layer B.Cu) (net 5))
 (segment (start 103.5 92.700002) (end 105.300001 94.500003) (width 0.25) (layer B.Cu) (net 5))
 (segment (start 105.300001 94.500003) (end 105.7 94.900002) (width 0.25) (layer B.Cu) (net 5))
 (segment (start 106.000002 94.6) (end 105.7 94.900002) (width 0.25) (layer F.Cu) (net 5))
 (segment (start 107.4 94.5) (end 107.3 94.6) (width 0.25) (layer F.Cu) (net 5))
 (segment (start 107.3 94.6) (end 106.000002 94.6) (width 0.25) (layer F.Cu) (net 5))
 (segment (start 100.5 94.515699) (end 100.5 95.4) (width 0.25) (layer F.Cu) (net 9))
 (segment (start 100.55001 94.134311) (end 100.55001 94.465689) (width 0.25) (layer F.Cu) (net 9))
 (segment (start 100.540699 94.125) (end 100.55001 94.134311) (width 0.25) (layer F.Cu) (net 9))
 (segment (start 100.55001 94.115689) (end 100.540699 94.125) (width 0.25) (layer F.Cu) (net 9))
 (segment (start 102.167001 84.478239) (end 102.167001 85.832999) (width 0.25) (layer F.Cu) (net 9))
 (segment (start 99.81 82.46) (end 100.571999 83.221999) (width 0.25) (layer F.Cu) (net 9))
 (segment (start 102.167001 85.832999) (end 100.5 87.5) (width 0.25) (layer F.Cu) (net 9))
 (segment (start 100.910761 83.221999) (end 102.167001 84.478239) (width 0.25) (layer F.Cu) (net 9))
 (segment (start 100.5 93.384301) (end 100.55001 93.434311) (width 0.25) (layer F.Cu) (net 9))
 (segment (start 100.540699 93.775) (end 100.55001 93.784311) (width 0.25) (layer F.Cu) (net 9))
 (segment (start 100.55001 94.465689) (end 100.5 94.515699) (width 0.25) (layer F.Cu) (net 9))
 (segment (start 100.5 87.5) (end 100.5 93.384301) (width 0.25) (layer F.Cu) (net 9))
 (segment (start 100.571999 83.221999) (end 100.910761 83.221999) (width 0.25) (layer F.Cu) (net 9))
 (segment (start 100.55001 93.784311) (end 100.55001 94.115689) (width 0.25) (layer F.Cu) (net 9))
 (segment (start 100.55001 93.434311) (end 100.55001 93.765689) (width 0.25) (layer F.Cu) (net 9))
 (segment (start 100.55001 93.765689) (end 100.540699 93.775) (width 0.25) (layer F.Cu) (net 9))
 (segment (start 100 91.15) (end 96.5 94.65) (width 0.25) (layer F.Cu) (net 11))
 (segment (start 96.5 94.65) (end 96.5 96.65) (width 0.25) (layer F.Cu) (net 11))
 (segment (start 100 86.08) (end 100 91.15) (width 0.25) (layer F.Cu) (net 11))
 (segment (start 101.08 85) (end 100 86.08) (width 0.25) (layer F.Cu) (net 11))
 (segment (start 102.5 96.65) (end 102.5 94.65) (width 0.25) (layer F.Cu) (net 12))
 (segment (start 102.5 94.65) (end 104.049989 93.100011) (width 0.25) (layer F.Cu) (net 12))
 (segment (start 105.398001 85.761999) (end 106.16 85) (width 0.25) (layer F.Cu) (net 12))
 (segment (start 104.049989 87.110011) (end 105.398001 85.761999) (width 0.25) (layer F.Cu) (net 12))
 (segment (start 104.049989 93.100011) (end 104.049989 87.110011) (width 0.25) (layer F.Cu) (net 12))
 (segment (start 102.35 83.53763) (end 102.35 82.46) (width 0.25) (layer B.Cu) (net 13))
 (segment (start 102.35 87.425) (end 102.35 83.53763) (width 0.25) (layer B.Cu) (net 13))
 (segment (start 102 87.775) (end 102.35 87.425) (width 0.25) (layer B.Cu) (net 13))
 (segment (start 102 88.2125) (end 102 87.775) (width 0.25) (layer B.Cu) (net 13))
 (segment (start 103.5 85.12) (end 103.62 85) (width 0.25) (layer B.Cu) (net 14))
 (segment (start 103.5 88.2125) (end 103.5 85.12) (width 0.25) (layer B.Cu) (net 14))
 (segment (start 107.247001 85.521761) (end 104.5 88.268762) (width 0.25) (layer F.Cu) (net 10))
 (segment (start 107.247001 83.739371) (end 107.247001 85.521761) (width 0.25) (layer F.Cu) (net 10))
 (segment (start 105.96763 82.46) (end 107.247001 83.739371) (width 0.25) (layer F.Cu) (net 10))
 (segment (start 104.5 88.268762) (end 104.5 96.65) (width 0.25) (layer F.Cu) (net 10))
 (segment (start 104.89 82.46) (end 105.96763 82.46) (width 0.25) (layer F.Cu) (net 10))
 (via (at 102.5 80) (size 0.8) (drill 0.4) (layers F.Cu B.Cu) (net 1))
 (via (at 102.5 78.5) (size 0.8) (drill 0.4) (layers F.Cu B.Cu) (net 1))
 (segment (start 102.5 80) (end 102.5 78.5) (width 0.25) (layer F.Cu) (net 1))
 (segment (start 102.5 78.5) (end 102.5 77.575) (width 0.25) (layer B.Cu) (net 1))
 (segment (start 104 80) (end 102.5 80) (width 0.25) (layer B.Cu) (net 1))
 (segment (start 107.840366 83.840366) (end 104 80) (width 0.25) (layer B.Cu) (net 1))
 (segment (start 107 92.5) (end 106.1 91.6) (width 0.25) (layer B.Cu) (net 1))
 (segment (start 108.9 92.5) (end 107 92.5) (width 0.25) (layer B.Cu) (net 1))
 (segment (start 106.1 89.7) (end 107.840366 87.959634) (width 0.25) (layer B.Cu) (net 1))
 (segment (start 106.1 91.6) (end 106.1 89.7) (width 0.25) (layer B.Cu) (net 1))
 (segment (start 107.840366 87.959634) (end 107.840366 83.840366) (width 0.25) (layer B.Cu) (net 1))
 (via (at 107 87.5) (size 0.8) (drill 0.4) (layers F.Cu B.Cu) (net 7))
 (via (at 109.5 87.5) (size 0.8) (drill 0.4) (layers F.Cu B.Cu) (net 7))
 (segment (start 107 87.5) (end 109.5 87.5) (width 0.25) (layer F.Cu) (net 7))
 (segment (start 109.5 74.51) (end 107.02 72.03) (width 0.25) (layer B.Cu) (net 7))
 (segment (start 109.5 87.5) (end 109.5 74.51) (width 0.25) (layer B.Cu) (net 7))
 (segment (start 108.9 94.5) (end 108.4 95) (width 0.25) (layer B.Cu) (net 7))
 (segment (start 108.4 95) (end 107.1 95) (width 0.25) (layer B.Cu) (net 7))
 (segment (start 105.649989 88.850011) (end 106.600001 87.899999) (width 0.25) (layer B.Cu) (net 7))
 (segment (start 106.600001 87.899999) (end 107 87.5) (width 0.25) (layer B.Cu) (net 7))
 (segment (start 107.1 95) (end 105.649989 93.549989) (width 0.25) (layer B.Cu) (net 7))
 (segment (start 105.649989 93.549989) (end 105.649989 88.850011) (width 0.25) (layer B.Cu) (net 7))
 (segment (start 99.837498 79.274998) (end 98.5 77.9375) (width 0.25) (layer B.Cu) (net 3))
 (segment (start 98.5 77.9375) (end 98.5 77.5) (width 0.25) (layer B.Cu) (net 3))
 (segment (start 108.6 83.6) (end 104.274998 79.274998) (width 0.25) (layer B.Cu) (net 3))
 (segment (start 104.274998 79.274998) (end 99.837498 79.274998) (width 0.25) (layer B.Cu) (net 3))
 (segment (start 108.6 90.5) (end 108.6 83.6) (width 0.25) (layer B.Cu) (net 3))
 (segment (start 98.490661 70.954999) (end 107.536001 70.954999) (width 0.25) (layer B.Cu) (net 8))
 (segment (start 96.355 72.03) (end 97.41566 72.03) (width 0.25) (layer B.Cu) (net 8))
 (segment (start 107.536001 70.954999) (end 110.5 73.918998) (width 0.25) (layer B.Cu) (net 8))
 (segment (start 97.41566 72.03) (end 98.490661 70.954999) (width 0.25) (layer B.Cu) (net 8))
 (segment (start 110.5 73.918998) (end 110.5 88) (width 0.25) (layer B.Cu) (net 8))
 (via (at 109.5 89) (size 0.8) (drill 0.4) (layers F.Cu B.Cu) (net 8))
 (segment (start 110.5 88) (end 109.5 89) (width 0.25) (layer B.Cu) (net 8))
 (segment (start 109.5 89.65) (end 108.65 90.5) (width 0.25) (layer F.Cu) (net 8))
 (segment (start 109.5 89) (end 109.5 89.65) (width 0.25) (layer F.Cu) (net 8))
 (segment (start 96 88.6) (end 96 85) (width 0.25) (layer B.Cu) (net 6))
 (segment (start 92.1 92.5) (end 96 88.6) (width 0.25) (layer B.Cu) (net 6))
 (segment (start 93.680732 93.961926) (end 93.680732 93.197175) (width 0.25) (layer B.Cu) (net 6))
 (segment (start 92.983557 92.5) (end 92.1 92.5) (width 0.25) (layer B.Cu) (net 6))
 (segment (start 92.642658 95) (end 93.680732 93.961926) (width 0.25) (layer B.Cu) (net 6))
 (segment (start 93.680732 93.197175) (end 92.983557 92.5) (width 0.25) (layer B.Cu) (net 6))
 (segment (start 92.6 95) (end 92.642658 95) (width 0.25) (layer B.Cu) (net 6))
 (segment (start 92.1 94.5) (end 92.6 95) (width 0.25) (layer B.Cu) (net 6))
 (segment (start 97.71 75.925) (end 93.815 72.03) (width 0.25) (layer B.Cu) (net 4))
 (segment (start 98.5 75.925) (end 97.71 75.925) (width 0.25) (layer B.Cu) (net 4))
 (segment (start 102.5 74.01) (end 104 72.51) (width 0.25) (layer B.Cu) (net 2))
 (segment (start 102.5 76) (end 102.5 74.01) (width 0.25) (layer B.Cu) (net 2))
 (segment (start 104 72.51) (end 104.48 72.03) (width 0.25) (layer B.Cu) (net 2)))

